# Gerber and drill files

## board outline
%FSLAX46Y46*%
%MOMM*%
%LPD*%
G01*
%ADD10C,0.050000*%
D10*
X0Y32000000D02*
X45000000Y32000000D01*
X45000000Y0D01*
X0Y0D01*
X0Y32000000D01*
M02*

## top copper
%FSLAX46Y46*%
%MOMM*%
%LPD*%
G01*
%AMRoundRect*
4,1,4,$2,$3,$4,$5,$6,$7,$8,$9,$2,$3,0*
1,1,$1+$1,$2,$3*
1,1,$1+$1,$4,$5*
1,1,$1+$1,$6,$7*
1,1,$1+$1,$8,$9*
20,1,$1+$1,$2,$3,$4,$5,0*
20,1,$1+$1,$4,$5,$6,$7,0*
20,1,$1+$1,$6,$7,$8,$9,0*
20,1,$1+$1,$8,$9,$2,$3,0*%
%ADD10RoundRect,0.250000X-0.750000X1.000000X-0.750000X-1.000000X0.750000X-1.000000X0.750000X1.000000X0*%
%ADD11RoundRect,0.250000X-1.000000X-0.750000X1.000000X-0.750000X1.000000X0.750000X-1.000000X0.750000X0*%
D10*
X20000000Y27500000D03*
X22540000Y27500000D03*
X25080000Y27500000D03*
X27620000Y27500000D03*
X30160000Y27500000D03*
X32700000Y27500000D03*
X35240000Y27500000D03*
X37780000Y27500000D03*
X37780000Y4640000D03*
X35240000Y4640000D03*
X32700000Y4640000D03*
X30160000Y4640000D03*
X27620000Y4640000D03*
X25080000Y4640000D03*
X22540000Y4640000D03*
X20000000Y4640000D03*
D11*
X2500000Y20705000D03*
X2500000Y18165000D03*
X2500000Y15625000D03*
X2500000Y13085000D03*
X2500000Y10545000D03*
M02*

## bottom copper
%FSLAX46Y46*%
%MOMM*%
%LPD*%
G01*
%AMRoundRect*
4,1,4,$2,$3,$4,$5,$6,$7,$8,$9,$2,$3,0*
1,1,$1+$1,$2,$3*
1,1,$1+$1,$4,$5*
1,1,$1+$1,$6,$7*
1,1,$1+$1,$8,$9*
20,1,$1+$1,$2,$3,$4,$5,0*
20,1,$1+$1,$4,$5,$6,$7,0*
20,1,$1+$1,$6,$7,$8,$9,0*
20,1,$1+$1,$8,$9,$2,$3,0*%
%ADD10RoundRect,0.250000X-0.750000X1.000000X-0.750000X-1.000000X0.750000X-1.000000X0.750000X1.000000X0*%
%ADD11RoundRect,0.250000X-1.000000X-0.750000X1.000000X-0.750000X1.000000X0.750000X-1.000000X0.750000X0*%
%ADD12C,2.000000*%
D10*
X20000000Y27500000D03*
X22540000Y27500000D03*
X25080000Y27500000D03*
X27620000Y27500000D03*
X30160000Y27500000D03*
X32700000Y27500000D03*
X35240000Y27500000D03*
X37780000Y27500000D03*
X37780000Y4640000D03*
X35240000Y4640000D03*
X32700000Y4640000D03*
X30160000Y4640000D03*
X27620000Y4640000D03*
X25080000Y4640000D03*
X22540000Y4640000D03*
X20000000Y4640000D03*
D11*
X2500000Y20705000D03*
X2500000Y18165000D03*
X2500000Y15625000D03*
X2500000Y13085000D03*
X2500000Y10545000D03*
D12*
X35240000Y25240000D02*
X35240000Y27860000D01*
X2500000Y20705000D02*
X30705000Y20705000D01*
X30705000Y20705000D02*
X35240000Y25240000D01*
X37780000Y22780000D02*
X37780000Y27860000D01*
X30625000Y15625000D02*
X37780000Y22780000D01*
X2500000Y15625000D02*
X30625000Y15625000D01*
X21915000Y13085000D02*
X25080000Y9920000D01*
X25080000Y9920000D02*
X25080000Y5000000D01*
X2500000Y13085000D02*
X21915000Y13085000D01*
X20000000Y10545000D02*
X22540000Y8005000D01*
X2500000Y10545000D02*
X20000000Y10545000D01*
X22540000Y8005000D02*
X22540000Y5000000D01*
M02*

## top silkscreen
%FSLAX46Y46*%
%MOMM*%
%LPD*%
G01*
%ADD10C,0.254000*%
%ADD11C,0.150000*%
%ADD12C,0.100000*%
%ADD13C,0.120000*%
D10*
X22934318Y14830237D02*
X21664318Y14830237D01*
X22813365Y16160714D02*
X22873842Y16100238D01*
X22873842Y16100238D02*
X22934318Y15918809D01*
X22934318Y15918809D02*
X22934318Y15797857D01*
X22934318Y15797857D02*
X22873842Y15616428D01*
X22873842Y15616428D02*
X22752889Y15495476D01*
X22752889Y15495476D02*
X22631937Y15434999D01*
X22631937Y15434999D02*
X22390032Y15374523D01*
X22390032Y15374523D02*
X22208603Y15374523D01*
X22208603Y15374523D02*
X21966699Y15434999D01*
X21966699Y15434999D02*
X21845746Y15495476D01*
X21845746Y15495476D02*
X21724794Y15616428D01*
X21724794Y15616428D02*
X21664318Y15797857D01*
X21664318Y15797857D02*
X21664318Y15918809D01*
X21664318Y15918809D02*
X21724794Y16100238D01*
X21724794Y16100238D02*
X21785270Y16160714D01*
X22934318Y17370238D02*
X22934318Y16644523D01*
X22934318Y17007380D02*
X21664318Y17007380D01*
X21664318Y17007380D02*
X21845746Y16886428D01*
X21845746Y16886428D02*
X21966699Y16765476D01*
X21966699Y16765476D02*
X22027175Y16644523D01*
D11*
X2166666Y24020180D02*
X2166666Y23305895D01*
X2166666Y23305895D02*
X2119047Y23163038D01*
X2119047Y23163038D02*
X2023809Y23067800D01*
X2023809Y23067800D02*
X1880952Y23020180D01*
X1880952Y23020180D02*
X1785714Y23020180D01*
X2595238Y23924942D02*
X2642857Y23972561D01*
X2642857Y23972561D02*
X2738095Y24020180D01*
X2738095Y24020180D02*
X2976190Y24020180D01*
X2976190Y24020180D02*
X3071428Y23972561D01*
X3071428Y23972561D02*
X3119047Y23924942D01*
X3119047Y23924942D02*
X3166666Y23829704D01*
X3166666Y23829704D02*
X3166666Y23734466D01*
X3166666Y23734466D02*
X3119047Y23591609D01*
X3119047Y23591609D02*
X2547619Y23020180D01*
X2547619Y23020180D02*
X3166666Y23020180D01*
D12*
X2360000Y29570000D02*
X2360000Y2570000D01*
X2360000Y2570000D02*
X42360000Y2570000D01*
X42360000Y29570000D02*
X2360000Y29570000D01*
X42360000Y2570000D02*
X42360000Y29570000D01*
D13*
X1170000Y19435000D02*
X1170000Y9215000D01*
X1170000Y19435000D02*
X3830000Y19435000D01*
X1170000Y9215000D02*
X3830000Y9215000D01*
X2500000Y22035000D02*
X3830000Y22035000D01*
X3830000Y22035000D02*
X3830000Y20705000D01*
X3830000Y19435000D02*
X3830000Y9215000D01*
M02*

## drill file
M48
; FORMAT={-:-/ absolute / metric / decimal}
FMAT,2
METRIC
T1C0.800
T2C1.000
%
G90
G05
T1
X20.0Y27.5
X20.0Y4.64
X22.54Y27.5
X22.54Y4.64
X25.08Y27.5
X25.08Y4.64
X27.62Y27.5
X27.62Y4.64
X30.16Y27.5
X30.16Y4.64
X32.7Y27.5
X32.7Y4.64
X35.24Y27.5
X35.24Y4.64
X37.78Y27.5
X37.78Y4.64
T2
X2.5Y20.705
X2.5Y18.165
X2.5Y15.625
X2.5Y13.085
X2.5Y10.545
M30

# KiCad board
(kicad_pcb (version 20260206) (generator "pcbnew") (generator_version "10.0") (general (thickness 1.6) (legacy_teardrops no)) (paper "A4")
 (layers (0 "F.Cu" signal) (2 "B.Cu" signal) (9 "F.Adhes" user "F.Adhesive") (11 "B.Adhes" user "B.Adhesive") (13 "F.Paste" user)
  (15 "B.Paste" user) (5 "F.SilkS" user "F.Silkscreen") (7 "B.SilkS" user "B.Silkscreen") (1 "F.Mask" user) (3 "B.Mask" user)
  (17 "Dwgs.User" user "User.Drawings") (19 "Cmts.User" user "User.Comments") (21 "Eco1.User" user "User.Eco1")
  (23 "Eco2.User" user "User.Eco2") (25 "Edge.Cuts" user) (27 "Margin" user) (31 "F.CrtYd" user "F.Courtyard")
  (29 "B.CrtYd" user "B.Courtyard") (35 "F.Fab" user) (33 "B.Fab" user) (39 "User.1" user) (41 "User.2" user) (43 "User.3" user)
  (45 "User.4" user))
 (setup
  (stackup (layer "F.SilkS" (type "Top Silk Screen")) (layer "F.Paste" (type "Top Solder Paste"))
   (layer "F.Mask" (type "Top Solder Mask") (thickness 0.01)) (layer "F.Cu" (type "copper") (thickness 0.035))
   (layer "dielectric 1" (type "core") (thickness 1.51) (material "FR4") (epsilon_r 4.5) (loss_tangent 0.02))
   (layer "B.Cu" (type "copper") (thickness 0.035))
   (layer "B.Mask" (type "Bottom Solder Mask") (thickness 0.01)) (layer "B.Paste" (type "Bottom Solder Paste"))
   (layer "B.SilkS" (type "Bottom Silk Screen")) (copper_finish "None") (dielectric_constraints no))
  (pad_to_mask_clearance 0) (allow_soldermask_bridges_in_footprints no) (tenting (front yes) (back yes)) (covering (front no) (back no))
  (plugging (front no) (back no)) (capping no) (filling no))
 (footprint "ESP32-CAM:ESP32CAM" (layer "F.Cu") (at 20 -27.5 -90)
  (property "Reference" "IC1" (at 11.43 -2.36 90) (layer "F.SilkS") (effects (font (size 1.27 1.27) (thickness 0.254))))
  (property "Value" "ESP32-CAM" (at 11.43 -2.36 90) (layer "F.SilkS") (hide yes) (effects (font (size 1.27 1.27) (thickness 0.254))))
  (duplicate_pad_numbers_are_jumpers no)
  (fp_line (start -2.07 17.64) (end 24.93 17.64) (stroke (width 0.1) (type solid)) (layer "F.SilkS"))
  (fp_line (start 24.93 17.64) (end 24.93 -22.36) (stroke (width 0.1) (type solid)) (layer "F.SilkS"))
  (fp_line (start -2.07 -22.36) (end -2.07 17.64) (stroke (width 0.1) (type solid)) (layer "F.SilkS"))
  (fp_line (start 24.93 -22.36) (end -2.07 -22.36) (stroke (width 0.1) (type solid)) (layer "F.SilkS"))
  (pad "1" thru_hole roundrect (at 0 0 270) (size 2.5 2) (drill 0.8) (layers "*.Cu" "*.Mask") (remove_unused_layers no)
   (roundrect_rratio 0.125) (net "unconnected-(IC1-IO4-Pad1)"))
  (pad "2" thru_hole roundrect (at 0 -2.54 270) (size 2.5 2) (drill 0.8) (layers "*.Cu" "*.Mask") (remove_unused_layers no)
   (roundrect_rratio 0.125) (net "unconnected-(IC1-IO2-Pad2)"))
  (pad "3" thru_hole roundrect (at 0 -5.08 270) (size 2.5 2) (drill 0.8) (layers "*.Cu" "*.Mask") (remove_unused_layers no)
   (roundrect_rratio 0.125) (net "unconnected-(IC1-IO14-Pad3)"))
  (pad "4" thru_hole roundrect (at 0 -7.62 270) (size 2.5 2) (drill 0.8) (layers "*.Cu" "*.Mask") (remove_unused_layers no)
   (roundrect_rratio 0.125) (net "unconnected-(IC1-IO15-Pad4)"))
  (pad "5" thru_hole roundrect (at 0 -10.16 270) (size 2.5 2) (drill 0.8) (layers "*.Cu" "*.Mask") (remove_unused_layers no)
   (roundrect_rratio 0.125) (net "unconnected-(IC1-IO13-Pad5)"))
  (pad "6" thru_hole roundrect (at 0 -12.7 270) (size 2.5 2) (drill 0.8) (layers "*.Cu" "*.Mask") (remove_unused_layers no)
   (roundrect_rratio 0.125) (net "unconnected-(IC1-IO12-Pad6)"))
  (pad "7" thru_hole roundrect (at 0 -15.24 270) (size 2.5 2) (drill 0.8) (layers "*.Cu" "*.Mask") (remove_unused_layers no)
   (roundrect_rratio 0.125) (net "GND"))
  (pad "8" thru_hole roundrect (at 0 -17.78 270) (size 2.5 2) (drill 0.8) (layers "*.Cu" "*.Mask") (remove_unused_layers no)
   (roundrect_rratio 0.125) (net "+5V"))
  (pad "9" thru_hole roundrect (at 22.86 -17.78 270) (size 2.5 2) (drill 0.8) (layers "*.Cu" "*.Mask") (remove_unused_layers no)
   (roundrect_rratio 0.125) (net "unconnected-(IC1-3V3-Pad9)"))
  (pad "10" thru_hole roundrect (at 22.86 -15.24 270) (size 2.5 2) (drill 0.8) (layers "*.Cu" "*.Mask") (remove_unused_layers no)
   (roundrect_rratio 0.125) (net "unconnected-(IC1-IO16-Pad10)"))
  (pad "11" thru_hole roundrect (at 22.86 -12.7 270) (size 2.5 2) (drill 0.8) (layers "*.Cu" "*.Mask") (remove_unused_layers no)
   (roundrect_rratio 0.125) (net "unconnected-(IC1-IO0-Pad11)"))
  (pad "12" thru_hole roundrect (at 22.86 -10.16 270) (size 2.5 2) (drill 0.8) (layers "*.Cu" "*.Mask") (remove_unused_layers no)
   (roundrect_rratio 0.125) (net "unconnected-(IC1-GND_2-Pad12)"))
  (pad "13" thru_hole roundrect (at 22.86 -7.62 270) (size 2.5 2) (drill 0.8) (layers "*.Cu" "*.Mask") (remove_unused_layers no)
   (roundrect_rratio 0.125) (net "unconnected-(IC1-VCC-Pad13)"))
  (pad "14" thru_hole roundrect (at 22.86 -5.08 270) (size 2.5 2) (drill 0.8) (layers "*.Cu" "*.Mask") (remove_unused_layers no)
   (roundrect_rratio 0.125) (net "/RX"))
  (pad "15" thru_hole roundrect (at 22.86 -2.54 270) (size 2.5 2) (drill 0.8) (layers "*.Cu" "*.Mask") (remove_unused_layers no)
   (roundrect_rratio 0.125) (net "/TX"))
  (pad "16" thru_hole roundrect (at 22.86 0 270) (size 2.5 2) (drill 0.8) (layers "*.Cu" "*.Mask") (remove_unused_layers no)
   (roundrect_rratio 0.125) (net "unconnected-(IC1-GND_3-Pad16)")))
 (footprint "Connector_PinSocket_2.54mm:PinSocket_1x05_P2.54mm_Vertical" (layer "F.Cu") (at 2.5 -20.705)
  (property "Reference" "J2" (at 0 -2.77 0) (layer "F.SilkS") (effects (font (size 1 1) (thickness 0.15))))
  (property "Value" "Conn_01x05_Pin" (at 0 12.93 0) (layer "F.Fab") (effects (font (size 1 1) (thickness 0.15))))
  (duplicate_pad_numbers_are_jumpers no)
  (fp_line (start -1.33 1.27) (end -1.33 11.49) (stroke (width 0.12) (type solid)) (layer "F.SilkS"))
  (fp_line (start -1.33 1.27) (end 1.33 1.27) (stroke (width 0.12) (type solid)) (layer "F.SilkS"))
  (fp_line (start -1.33 11.49) (end 1.33 11.49) (stroke (width 0.12) (type solid)) (layer "F.SilkS"))
  (fp_line (start 0 -1.33) (end 1.33 -1.33) (stroke (width 0.12) (type solid)) (layer "F.SilkS"))
  (fp_line (start 1.33 -1.33) (end 1.33 0) (stroke (width 0.12) (type solid)) (layer "F.SilkS"))
  (fp_line (start 1.33 1.27) (end 1.33 11.49) (stroke (width 0.12) (type solid)) (layer "F.SilkS"))
  (pad "1" thru_hole roundrect (at 0 0) (size 2.5 2) (drill 1) (layers "*.Cu" "*.Mask") (remove_unused_layers no) (roundrect_rratio 0.125)
   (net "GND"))
  (pad "2" thru_hole roundrect (at 0 2.54) (size 2.5 2) (drill 1) (layers "*.Cu" "*.Mask") (remove_unused_layers no)
   (roundrect_rratio 0.125) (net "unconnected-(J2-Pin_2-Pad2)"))
  (pad "3" thru_hole roundrect (at 0 5.08) (size 2.5 2) (drill 1) (layers "*.Cu" "*.Mask") (remove_unused_layers no)
   (roundrect_rratio 0.125) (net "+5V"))
  (pad "4" thru_hole roundrect (at 0 7.62) (size 2.5 2) (drill 1) (layers "*.Cu" "*.Mask") (remove_unused_layers no)
   (roundrect_rratio 0.125) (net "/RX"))
  (pad "5" thru_hole roundrect (at 0 10.16) (size 2.5 2) (drill 1) (layers "*.Cu" "*.Mask") (remove_unused_layers no)
   (roundrect_rratio 0.125) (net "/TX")))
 (gr_rect (start 0 -32) (end 45 0) (stroke (width 0.05) (type default)) (fill no) (layer "Edge.Cuts"))
 (segment (start 35.24 -25.24) (end 35.24 -27.86) (width 2) (layer "B.Cu") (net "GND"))
 (segment (start 2.5 -20.705) (end 30.705 -20.705) (width 2) (layer "B.Cu") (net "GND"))
 (segment (start 30.705 -20.705) (end 35.24 -25.24) (width 2) (layer "B.Cu") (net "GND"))
 (segment (start 37.78 -22.78) (end 37.78 -27.86) (width 2) (layer "B.Cu") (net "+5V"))
 (segment (start 30.625 -15.625) (end 37.78 -22.78) (width 2) (layer "B.Cu") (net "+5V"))
 (segment (start 2.5 -15.625) (end 30.625 -15.625) (width 2) (layer "B.Cu") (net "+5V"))
 (segment (start 21.915 -13.085) (end 25.08 -9.92) (width 2) (layer "B.Cu") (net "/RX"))
 (segment (start 25.08 -9.92) (end 25.08 -5) (width 2) (layer "B.Cu") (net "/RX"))
 (segment (start 2.5 -13.085) (end 21.915 -13.085) (width 2) (layer "B.Cu") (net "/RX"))
 (segment (start 20 -10.545) (end 22.54 -8.005) (width 2) (layer "B.Cu") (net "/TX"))
 (segment (start 2.5 -10.545) (end 20 -10.545) (width 2) (layer "B.Cu") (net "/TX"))
 (segment (start 22.54 -8.005) (end 22.54 -5) (width 2) (layer "B.Cu") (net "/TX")))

